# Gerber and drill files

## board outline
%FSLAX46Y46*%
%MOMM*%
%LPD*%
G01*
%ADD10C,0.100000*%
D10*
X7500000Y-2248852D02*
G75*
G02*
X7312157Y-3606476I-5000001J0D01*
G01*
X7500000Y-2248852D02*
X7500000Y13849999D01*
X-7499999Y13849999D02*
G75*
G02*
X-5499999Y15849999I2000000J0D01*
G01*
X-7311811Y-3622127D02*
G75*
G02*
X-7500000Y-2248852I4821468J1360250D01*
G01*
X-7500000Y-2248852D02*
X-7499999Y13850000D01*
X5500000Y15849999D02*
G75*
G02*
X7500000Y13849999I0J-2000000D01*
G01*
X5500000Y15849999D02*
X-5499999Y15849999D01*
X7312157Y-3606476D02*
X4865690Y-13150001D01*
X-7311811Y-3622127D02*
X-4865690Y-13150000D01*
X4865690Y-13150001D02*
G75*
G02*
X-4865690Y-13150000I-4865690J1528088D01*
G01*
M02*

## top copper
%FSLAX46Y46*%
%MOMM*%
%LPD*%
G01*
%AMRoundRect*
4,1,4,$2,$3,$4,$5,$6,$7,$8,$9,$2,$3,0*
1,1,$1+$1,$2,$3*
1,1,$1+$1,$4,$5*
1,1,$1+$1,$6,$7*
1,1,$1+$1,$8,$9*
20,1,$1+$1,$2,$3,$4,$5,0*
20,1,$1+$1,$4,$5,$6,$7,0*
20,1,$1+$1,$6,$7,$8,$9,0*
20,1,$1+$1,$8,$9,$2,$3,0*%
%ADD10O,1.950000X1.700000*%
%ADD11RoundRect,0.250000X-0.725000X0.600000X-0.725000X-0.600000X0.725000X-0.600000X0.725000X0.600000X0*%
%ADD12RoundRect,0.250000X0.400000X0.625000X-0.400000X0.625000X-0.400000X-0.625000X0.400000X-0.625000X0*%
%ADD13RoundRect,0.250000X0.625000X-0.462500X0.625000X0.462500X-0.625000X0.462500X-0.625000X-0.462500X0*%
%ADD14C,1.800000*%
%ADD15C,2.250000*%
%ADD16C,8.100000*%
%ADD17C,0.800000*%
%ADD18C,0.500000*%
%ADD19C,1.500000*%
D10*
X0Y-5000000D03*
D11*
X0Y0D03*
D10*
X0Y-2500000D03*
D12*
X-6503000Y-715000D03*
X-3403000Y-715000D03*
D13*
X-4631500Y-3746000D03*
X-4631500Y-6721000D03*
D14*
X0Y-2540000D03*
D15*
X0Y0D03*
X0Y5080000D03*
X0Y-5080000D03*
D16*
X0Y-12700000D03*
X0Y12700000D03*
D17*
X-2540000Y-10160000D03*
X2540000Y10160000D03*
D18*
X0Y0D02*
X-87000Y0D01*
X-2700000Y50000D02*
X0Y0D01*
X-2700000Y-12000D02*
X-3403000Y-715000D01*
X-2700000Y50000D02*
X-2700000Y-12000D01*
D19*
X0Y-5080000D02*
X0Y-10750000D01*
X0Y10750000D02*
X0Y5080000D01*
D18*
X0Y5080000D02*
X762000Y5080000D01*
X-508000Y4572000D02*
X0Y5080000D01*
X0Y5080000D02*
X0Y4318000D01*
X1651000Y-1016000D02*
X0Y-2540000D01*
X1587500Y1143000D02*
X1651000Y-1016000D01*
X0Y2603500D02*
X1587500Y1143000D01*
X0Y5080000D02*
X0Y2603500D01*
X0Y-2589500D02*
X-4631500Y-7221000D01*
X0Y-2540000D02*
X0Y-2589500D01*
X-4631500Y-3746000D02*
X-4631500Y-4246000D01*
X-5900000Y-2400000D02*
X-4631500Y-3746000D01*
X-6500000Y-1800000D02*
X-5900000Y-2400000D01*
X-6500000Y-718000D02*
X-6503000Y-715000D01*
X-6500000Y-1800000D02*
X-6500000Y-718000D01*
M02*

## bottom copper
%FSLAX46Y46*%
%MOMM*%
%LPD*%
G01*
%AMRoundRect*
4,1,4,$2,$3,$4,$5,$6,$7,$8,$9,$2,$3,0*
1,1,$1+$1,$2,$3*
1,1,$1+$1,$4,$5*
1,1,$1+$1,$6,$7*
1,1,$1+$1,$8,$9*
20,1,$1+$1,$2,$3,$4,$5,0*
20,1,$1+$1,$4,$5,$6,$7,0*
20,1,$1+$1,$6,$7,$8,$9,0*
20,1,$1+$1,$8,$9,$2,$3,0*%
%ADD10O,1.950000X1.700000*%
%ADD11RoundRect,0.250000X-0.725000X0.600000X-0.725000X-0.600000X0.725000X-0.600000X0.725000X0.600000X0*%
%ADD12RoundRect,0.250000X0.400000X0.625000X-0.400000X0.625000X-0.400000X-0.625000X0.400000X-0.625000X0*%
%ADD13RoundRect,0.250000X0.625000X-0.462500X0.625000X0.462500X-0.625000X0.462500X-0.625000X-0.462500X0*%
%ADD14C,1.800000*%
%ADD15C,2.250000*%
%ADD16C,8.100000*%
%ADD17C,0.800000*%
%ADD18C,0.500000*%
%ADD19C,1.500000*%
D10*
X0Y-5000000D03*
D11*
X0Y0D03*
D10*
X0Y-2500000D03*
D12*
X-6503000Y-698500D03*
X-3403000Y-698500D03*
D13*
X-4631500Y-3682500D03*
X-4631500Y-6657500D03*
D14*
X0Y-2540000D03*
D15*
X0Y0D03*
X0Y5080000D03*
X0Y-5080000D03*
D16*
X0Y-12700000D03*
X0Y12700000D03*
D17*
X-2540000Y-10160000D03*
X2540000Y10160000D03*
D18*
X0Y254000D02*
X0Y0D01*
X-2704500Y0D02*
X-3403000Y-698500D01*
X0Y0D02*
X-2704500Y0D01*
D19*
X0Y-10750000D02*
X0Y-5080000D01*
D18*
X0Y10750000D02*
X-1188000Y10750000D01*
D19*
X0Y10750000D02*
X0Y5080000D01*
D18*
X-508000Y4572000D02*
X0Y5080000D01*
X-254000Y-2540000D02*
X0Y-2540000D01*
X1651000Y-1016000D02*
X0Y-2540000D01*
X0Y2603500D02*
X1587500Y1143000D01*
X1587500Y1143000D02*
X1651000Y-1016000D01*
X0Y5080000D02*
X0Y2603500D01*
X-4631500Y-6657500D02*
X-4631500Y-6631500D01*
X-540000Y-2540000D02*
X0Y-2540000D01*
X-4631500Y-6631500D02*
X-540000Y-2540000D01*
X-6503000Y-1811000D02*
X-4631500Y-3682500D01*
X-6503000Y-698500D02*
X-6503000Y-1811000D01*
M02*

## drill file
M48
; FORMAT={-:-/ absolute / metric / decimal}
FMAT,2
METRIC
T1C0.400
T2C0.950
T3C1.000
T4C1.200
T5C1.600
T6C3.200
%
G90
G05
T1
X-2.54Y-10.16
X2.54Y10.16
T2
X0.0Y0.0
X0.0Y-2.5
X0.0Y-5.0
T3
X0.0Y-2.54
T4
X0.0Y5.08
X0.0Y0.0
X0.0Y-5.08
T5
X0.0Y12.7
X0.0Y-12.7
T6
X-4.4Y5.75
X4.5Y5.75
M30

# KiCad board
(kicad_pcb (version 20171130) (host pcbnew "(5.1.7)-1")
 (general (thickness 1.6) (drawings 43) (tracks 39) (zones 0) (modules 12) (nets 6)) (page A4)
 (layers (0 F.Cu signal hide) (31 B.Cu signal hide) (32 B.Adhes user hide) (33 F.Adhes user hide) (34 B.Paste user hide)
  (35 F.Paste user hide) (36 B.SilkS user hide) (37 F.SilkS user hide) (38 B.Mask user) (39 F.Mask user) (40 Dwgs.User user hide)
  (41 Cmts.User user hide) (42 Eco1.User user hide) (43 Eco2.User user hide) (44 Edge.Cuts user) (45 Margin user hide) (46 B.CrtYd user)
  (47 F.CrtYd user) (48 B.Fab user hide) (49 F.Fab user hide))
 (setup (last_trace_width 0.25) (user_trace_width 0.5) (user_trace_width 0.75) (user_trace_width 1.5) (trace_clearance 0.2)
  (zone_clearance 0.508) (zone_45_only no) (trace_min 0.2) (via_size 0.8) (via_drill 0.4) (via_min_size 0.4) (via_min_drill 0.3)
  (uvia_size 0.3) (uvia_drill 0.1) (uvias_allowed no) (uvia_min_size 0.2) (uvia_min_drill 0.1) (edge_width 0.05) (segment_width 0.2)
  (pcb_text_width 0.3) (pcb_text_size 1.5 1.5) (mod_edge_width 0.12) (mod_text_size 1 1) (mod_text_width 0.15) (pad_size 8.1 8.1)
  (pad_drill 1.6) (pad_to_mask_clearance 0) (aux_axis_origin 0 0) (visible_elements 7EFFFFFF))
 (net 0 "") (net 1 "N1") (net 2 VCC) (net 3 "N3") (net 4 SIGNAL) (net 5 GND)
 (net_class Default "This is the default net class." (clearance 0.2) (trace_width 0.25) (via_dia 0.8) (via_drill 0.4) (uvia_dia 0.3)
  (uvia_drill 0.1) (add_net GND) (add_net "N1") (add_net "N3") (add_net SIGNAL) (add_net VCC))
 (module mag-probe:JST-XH (layer F.Cu) (at 0 0 270)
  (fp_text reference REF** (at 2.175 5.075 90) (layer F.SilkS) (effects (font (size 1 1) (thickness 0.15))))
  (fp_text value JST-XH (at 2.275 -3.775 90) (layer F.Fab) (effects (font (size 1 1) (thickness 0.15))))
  (pad 3 thru_hole oval (at 5 0 270) (size 1.7 1.95) (drill 0.95) (layers *.Cu *.Mask))
  (pad 1 thru_hole roundrect (at 0 0 270) (size 1.7 1.95) (drill 0.95) (layers *.Cu *.Mask) (roundrect_rratio 0.147059))
  (pad 2 thru_hole oval (at 2.5 0 270) (size 1.7 1.95) (drill 0.95) (layers *.Cu *.Mask)))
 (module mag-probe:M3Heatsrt (layer F.Cu) (at -4.45 -5.8)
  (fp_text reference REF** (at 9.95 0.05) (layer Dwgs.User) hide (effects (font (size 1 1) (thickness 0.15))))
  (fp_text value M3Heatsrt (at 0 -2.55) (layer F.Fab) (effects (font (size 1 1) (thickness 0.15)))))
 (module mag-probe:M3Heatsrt (layer F.Cu) (at 4.45 -5.85)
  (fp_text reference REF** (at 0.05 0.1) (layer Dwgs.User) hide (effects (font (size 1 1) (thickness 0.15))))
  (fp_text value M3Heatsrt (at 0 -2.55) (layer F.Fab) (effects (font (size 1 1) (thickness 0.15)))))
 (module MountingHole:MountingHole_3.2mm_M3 (layer F.Cu) (at -4.5 -5.75)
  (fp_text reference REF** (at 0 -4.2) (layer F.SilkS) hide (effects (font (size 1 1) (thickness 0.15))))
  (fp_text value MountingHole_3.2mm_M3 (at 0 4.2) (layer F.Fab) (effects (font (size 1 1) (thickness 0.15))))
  (pad "" np_thru_hole circle (at 0.1 0) (size 3.2 3.2) (drill 3.2) (layers *.Cu *.Mask)))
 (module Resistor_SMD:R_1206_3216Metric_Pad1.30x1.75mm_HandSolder (layer F.Cu) (at -4.953 0.715 180)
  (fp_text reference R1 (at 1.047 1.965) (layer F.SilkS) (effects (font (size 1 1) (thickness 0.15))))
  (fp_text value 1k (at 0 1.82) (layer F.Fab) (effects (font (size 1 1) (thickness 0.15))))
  (pad 2 smd roundrect (at 1.55 0 180) (size 1.3 1.75) (layers F.Cu F.Paste F.Mask) (roundrect_rratio 0.1923076923076923) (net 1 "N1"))
  (pad 1 smd roundrect (at -1.55 0 180) (size 1.3 1.75) (layers F.Cu F.Paste F.Mask) (roundrect_rratio 0.1923076923076923) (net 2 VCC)))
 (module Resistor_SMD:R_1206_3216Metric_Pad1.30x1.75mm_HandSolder (layer B.Cu) (at -4.953 0.6985 180)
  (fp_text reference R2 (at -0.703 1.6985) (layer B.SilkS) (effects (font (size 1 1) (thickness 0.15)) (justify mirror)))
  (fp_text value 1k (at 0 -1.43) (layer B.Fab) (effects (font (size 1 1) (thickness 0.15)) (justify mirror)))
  (pad 2 smd roundrect (at 1.55 0 180) (size 1.3 1.75) (layers B.Cu B.Paste B.Mask) (roundrect_rratio 0.1923076923076923) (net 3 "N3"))
  (pad 1 smd roundrect (at -1.55 0 180) (size 1.3 1.75) (layers B.Cu B.Paste B.Mask) (roundrect_rratio 0.1923076923076923) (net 2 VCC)))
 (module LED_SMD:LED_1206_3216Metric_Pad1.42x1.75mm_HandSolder (layer F.Cu) (at -4.6315 5.2335 90)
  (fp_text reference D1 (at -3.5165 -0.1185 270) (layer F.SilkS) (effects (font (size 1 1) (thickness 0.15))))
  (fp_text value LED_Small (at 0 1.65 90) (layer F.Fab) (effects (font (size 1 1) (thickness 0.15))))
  (pad 2 smd roundrect (at 1.4875 0 90) (size 1.425 1.75) (layers F.Cu F.Paste F.Mask) (roundrect_rratio 0.1754385964912281) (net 1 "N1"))
  (pad 1 smd roundrect (at -1.4875 0 90) (size 1.425 1.75) (layers F.Cu F.Paste F.Mask) (roundrect_rratio 0.1754385964912281) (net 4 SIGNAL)))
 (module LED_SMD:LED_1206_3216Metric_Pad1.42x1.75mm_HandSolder (layer B.Cu) (at -4.6315 5.17 90)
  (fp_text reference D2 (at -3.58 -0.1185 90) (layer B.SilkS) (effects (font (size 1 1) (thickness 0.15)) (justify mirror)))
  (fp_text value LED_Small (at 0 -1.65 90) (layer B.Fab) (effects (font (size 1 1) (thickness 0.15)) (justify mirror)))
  (pad 2 smd roundrect (at 1.4875 0 90) (size 1.425 1.75) (layers B.Cu B.Paste B.Mask) (roundrect_rratio 0.1754385964912281) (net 3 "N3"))
  (pad 1 smd roundrect (at -1.4875 0 90) (size 1.425 1.75) (layers B.Cu B.Paste B.Mask) (roundrect_rratio 0.1754385964912281) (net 4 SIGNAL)))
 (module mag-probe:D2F (layer F.Cu) (at 0 0 270)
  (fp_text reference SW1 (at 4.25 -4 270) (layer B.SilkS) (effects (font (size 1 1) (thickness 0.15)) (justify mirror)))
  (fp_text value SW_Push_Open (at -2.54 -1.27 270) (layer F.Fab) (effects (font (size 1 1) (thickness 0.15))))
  (pad 4 thru_hole circle (at 2.54 0 270) (size 1.8 1.8) (drill 1) (layers *.Cu *.Mask) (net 4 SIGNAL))
  (pad 3 thru_hole circle (at 0 0 270) (size 2.25 2.25) (drill 1.2) (layers *.Cu *.Mask) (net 2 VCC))
  (pad 2 thru_hole circle (at -5.08 0 270) (size 2.25 2.25) (drill 1.2) (layers *.Cu *.Mask) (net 4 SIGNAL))
  (pad 1 thru_hole circle (at 5.08 0 270) (size 2.25 2.25) (drill 1.2) (layers *.Cu *.Mask) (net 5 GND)))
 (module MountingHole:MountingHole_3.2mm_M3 (layer F.Cu) (at 4.5 -5.75)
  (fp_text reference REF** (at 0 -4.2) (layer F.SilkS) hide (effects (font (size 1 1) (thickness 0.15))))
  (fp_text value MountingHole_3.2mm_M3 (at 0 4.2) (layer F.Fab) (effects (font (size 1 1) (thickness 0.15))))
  (pad 1 np_thru_hole circle (at 0 0) (size 3.2 3.2) (drill 3.2) (layers *.Cu *.Mask)))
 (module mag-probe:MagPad (layer F.Cu) (at 0 12.7)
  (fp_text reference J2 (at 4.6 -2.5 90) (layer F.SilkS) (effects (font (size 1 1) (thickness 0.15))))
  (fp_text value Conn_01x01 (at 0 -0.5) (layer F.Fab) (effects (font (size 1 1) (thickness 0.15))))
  (pad 1 thru_hole circle (at 0 0) (size 8.1 8.1) (drill 1.6) (layers *.Cu *.Mask) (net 5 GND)))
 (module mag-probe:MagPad (layer F.Cu) (at 0 -12.7)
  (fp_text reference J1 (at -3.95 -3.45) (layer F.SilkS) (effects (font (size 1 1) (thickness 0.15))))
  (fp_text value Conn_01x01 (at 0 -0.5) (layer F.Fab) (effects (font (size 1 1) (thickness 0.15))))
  (pad 1 thru_hole circle (at 0 0) (size 8.1 8.1) (drill 1.6) (layers *.Cu *.Mask) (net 4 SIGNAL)))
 (gr_arc (start 2.499999 2.248852) (end 7.312157 3.606476) (angle -15.75501346) (layer Edge.Cuts) (width 0.1))
 (gr_line (start 7.5 2.248852) (end 7.5 -13.849999) (layer Edge.Cuts) (width 0.1))
 (gr_arc (start -5.499999 -13.849999) (end -5.499999 -15.849999) (angle -90) (layer Edge.Cuts) (width 0.1))
 (gr_arc (start -2.490343 2.261877) (end -7.5 2.248852) (angle -15.90398022) (layer Edge.Cuts) (width 0.1))
 (gr_line (start -7.5 2.248852) (end -7.499999 -13.85) (layer Edge.Cuts) (width 0.1))
 (gr_arc (start 5.5 -13.849999) (end 7.5 -13.849999) (angle -90) (layer Edge.Cuts) (width 0.1))
 (gr_line (start 5.5 -15.849999) (end -5.499999 -15.849999) (layer Edge.Cuts) (width 0.1))
 (gr_line (start 7.312157 3.606476) (end 4.86569 13.150001) (layer Edge.Cuts) (width 0.1))
 (gr_line (start -7.311811 3.622127) (end -4.86569 13.15) (layer Edge.Cuts) (width 0.1))
 (gr_arc (start 0 11.621913) (end -4.86569 13.15) (angle -145.1298326) (layer Edge.Cuts) (width 0.1))
 (segment (start 0 -0.254) (end 0 0) (width 0.5) (layer B.Cu) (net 2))
 (segment (start 0 0) (end -0.087 0) (width 0.5) (layer F.Cu) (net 2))
 (segment (start -2.7045 0) (end -3.403 0.6985) (width 0.5) (layer B.Cu) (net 2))
 (segment (start 0 0) (end -2.7045 0) (width 0.5) (layer B.Cu) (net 2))
 (segment (start -2.7 -0.05) (end 0 0) (width 0.5) (layer F.Cu) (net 2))
 (segment (start -2.7 0.012) (end -3.403 0.715) (width 0.5) (layer F.Cu) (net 2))
 (segment (start -2.7 -0.05) (end -2.7 0.012) (width 0.5) (layer F.Cu) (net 2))
 (segment (start 0 10.75) (end 0 5.08) (width 1.5) (layer B.Cu) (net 5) (status 30))
 (segment (start 0 5.08) (end 0 10.75) (width 1.5) (layer F.Cu) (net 5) (status 30))
 (via (at -2.54 10.16) (size 0.8) (drill 0.4) (layers F.Cu B.Cu) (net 5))
 (via (at 2.54 -10.16) (size 0.8) (drill 0.4) (layers F.Cu B.Cu) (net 4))
 (segment (start 0 -10.75) (end -1.188 -10.75) (width 0.5) (layer B.Cu) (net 4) (status 30))
 (segment (start 0 -10.75) (end 0 -5.08) (width 1.5) (layer B.Cu) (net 4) (status 30))
 (segment (start -0.508 -4.572) (end 0 -5.08) (width 0.5) (layer B.Cu) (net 4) (status 30))
 (segment (start 0 -10.75) (end 0 -5.08) (width 1.5) (layer F.Cu) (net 4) (status 30))
 (segment (start 0 -5.08) (end 0.762 -5.08) (width 0.5) (layer F.Cu) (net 4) (status 30))
 (segment (start -0.508 -4.572) (end 0 -5.08) (width 0.5) (layer F.Cu) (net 4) (status 30))
 (segment (start -0.254 2.54) (end 0 2.54) (width 0.5) (layer B.Cu) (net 4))
 (segment (start 0 -5.08) (end 0 -4.318) (width 0.5) (layer F.Cu) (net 4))
 (segment (start 1.651 1.016) (end 0 2.54) (width 0.5) (layer F.Cu) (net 4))
 (segment (start 1.5875 -1.143) (end 1.651 1.016) (width 0.5) (layer F.Cu) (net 4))
 (segment (start 0 -2.6035) (end 1.5875 -1.143) (width 0.5) (layer F.Cu) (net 4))
 (segment (start 1.651 1.016) (end 0 2.54) (width 0.5) (layer B.Cu) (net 4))
 (segment (start 0 -2.6035) (end 1.5875 -1.143) (width 0.5) (layer B.Cu) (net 4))
 (segment (start 1.5875 -1.143) (end 1.651 1.016) (width 0.5) (layer B.Cu) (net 4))
 (segment (start 0 -5.08) (end 0 -2.6035) (width 0.5) (layer B.Cu) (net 4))
 (segment (start 0 -5.08) (end 0 -2.6035) (width 0.5) (layer F.Cu) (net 4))
 (segment (start 0 2.5895) (end -4.6315 7.221) (width 0.5) (layer F.Cu) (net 4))
 (segment (start 0 2.54) (end 0 2.5895) (width 0.5) (layer F.Cu) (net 4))
 (segment (start -4.6315 6.6575) (end -4.6315 6.6315) (width 0.5) (layer B.Cu) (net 4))
 (segment (start -0.54 2.54) (end 0 2.54) (width 0.5) (layer B.Cu) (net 4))
 (segment (start -4.6315 6.6315) (end -0.54 2.54) (width 0.5) (layer B.Cu) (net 4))
 (segment (start -4.6315 3.746) (end -4.6315 4.246) (width 0.5) (layer F.Cu) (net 1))
 (segment (start -5.9 2.4) (end -4.6315 3.746) (width 0.5) (layer F.Cu) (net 1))
 (segment (start -6.5 1.8) (end -5.9 2.4) (width 0.5) (layer F.Cu) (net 1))
 (segment (start -6.5 0.718) (end -6.503 0.715) (width 0.5) (layer F.Cu) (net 1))
 (segment (start -6.5 1.8) (end -6.5 0.718) (width 0.5) (layer F.Cu) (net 1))
 (segment (start -6.503 1.811) (end -4.6315 3.6825) (width 0.5) (layer B.Cu) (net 3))
 (segment (start -6.503 0.6985) (end -6.503 1.811) (width 0.5) (layer B.Cu) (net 3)))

